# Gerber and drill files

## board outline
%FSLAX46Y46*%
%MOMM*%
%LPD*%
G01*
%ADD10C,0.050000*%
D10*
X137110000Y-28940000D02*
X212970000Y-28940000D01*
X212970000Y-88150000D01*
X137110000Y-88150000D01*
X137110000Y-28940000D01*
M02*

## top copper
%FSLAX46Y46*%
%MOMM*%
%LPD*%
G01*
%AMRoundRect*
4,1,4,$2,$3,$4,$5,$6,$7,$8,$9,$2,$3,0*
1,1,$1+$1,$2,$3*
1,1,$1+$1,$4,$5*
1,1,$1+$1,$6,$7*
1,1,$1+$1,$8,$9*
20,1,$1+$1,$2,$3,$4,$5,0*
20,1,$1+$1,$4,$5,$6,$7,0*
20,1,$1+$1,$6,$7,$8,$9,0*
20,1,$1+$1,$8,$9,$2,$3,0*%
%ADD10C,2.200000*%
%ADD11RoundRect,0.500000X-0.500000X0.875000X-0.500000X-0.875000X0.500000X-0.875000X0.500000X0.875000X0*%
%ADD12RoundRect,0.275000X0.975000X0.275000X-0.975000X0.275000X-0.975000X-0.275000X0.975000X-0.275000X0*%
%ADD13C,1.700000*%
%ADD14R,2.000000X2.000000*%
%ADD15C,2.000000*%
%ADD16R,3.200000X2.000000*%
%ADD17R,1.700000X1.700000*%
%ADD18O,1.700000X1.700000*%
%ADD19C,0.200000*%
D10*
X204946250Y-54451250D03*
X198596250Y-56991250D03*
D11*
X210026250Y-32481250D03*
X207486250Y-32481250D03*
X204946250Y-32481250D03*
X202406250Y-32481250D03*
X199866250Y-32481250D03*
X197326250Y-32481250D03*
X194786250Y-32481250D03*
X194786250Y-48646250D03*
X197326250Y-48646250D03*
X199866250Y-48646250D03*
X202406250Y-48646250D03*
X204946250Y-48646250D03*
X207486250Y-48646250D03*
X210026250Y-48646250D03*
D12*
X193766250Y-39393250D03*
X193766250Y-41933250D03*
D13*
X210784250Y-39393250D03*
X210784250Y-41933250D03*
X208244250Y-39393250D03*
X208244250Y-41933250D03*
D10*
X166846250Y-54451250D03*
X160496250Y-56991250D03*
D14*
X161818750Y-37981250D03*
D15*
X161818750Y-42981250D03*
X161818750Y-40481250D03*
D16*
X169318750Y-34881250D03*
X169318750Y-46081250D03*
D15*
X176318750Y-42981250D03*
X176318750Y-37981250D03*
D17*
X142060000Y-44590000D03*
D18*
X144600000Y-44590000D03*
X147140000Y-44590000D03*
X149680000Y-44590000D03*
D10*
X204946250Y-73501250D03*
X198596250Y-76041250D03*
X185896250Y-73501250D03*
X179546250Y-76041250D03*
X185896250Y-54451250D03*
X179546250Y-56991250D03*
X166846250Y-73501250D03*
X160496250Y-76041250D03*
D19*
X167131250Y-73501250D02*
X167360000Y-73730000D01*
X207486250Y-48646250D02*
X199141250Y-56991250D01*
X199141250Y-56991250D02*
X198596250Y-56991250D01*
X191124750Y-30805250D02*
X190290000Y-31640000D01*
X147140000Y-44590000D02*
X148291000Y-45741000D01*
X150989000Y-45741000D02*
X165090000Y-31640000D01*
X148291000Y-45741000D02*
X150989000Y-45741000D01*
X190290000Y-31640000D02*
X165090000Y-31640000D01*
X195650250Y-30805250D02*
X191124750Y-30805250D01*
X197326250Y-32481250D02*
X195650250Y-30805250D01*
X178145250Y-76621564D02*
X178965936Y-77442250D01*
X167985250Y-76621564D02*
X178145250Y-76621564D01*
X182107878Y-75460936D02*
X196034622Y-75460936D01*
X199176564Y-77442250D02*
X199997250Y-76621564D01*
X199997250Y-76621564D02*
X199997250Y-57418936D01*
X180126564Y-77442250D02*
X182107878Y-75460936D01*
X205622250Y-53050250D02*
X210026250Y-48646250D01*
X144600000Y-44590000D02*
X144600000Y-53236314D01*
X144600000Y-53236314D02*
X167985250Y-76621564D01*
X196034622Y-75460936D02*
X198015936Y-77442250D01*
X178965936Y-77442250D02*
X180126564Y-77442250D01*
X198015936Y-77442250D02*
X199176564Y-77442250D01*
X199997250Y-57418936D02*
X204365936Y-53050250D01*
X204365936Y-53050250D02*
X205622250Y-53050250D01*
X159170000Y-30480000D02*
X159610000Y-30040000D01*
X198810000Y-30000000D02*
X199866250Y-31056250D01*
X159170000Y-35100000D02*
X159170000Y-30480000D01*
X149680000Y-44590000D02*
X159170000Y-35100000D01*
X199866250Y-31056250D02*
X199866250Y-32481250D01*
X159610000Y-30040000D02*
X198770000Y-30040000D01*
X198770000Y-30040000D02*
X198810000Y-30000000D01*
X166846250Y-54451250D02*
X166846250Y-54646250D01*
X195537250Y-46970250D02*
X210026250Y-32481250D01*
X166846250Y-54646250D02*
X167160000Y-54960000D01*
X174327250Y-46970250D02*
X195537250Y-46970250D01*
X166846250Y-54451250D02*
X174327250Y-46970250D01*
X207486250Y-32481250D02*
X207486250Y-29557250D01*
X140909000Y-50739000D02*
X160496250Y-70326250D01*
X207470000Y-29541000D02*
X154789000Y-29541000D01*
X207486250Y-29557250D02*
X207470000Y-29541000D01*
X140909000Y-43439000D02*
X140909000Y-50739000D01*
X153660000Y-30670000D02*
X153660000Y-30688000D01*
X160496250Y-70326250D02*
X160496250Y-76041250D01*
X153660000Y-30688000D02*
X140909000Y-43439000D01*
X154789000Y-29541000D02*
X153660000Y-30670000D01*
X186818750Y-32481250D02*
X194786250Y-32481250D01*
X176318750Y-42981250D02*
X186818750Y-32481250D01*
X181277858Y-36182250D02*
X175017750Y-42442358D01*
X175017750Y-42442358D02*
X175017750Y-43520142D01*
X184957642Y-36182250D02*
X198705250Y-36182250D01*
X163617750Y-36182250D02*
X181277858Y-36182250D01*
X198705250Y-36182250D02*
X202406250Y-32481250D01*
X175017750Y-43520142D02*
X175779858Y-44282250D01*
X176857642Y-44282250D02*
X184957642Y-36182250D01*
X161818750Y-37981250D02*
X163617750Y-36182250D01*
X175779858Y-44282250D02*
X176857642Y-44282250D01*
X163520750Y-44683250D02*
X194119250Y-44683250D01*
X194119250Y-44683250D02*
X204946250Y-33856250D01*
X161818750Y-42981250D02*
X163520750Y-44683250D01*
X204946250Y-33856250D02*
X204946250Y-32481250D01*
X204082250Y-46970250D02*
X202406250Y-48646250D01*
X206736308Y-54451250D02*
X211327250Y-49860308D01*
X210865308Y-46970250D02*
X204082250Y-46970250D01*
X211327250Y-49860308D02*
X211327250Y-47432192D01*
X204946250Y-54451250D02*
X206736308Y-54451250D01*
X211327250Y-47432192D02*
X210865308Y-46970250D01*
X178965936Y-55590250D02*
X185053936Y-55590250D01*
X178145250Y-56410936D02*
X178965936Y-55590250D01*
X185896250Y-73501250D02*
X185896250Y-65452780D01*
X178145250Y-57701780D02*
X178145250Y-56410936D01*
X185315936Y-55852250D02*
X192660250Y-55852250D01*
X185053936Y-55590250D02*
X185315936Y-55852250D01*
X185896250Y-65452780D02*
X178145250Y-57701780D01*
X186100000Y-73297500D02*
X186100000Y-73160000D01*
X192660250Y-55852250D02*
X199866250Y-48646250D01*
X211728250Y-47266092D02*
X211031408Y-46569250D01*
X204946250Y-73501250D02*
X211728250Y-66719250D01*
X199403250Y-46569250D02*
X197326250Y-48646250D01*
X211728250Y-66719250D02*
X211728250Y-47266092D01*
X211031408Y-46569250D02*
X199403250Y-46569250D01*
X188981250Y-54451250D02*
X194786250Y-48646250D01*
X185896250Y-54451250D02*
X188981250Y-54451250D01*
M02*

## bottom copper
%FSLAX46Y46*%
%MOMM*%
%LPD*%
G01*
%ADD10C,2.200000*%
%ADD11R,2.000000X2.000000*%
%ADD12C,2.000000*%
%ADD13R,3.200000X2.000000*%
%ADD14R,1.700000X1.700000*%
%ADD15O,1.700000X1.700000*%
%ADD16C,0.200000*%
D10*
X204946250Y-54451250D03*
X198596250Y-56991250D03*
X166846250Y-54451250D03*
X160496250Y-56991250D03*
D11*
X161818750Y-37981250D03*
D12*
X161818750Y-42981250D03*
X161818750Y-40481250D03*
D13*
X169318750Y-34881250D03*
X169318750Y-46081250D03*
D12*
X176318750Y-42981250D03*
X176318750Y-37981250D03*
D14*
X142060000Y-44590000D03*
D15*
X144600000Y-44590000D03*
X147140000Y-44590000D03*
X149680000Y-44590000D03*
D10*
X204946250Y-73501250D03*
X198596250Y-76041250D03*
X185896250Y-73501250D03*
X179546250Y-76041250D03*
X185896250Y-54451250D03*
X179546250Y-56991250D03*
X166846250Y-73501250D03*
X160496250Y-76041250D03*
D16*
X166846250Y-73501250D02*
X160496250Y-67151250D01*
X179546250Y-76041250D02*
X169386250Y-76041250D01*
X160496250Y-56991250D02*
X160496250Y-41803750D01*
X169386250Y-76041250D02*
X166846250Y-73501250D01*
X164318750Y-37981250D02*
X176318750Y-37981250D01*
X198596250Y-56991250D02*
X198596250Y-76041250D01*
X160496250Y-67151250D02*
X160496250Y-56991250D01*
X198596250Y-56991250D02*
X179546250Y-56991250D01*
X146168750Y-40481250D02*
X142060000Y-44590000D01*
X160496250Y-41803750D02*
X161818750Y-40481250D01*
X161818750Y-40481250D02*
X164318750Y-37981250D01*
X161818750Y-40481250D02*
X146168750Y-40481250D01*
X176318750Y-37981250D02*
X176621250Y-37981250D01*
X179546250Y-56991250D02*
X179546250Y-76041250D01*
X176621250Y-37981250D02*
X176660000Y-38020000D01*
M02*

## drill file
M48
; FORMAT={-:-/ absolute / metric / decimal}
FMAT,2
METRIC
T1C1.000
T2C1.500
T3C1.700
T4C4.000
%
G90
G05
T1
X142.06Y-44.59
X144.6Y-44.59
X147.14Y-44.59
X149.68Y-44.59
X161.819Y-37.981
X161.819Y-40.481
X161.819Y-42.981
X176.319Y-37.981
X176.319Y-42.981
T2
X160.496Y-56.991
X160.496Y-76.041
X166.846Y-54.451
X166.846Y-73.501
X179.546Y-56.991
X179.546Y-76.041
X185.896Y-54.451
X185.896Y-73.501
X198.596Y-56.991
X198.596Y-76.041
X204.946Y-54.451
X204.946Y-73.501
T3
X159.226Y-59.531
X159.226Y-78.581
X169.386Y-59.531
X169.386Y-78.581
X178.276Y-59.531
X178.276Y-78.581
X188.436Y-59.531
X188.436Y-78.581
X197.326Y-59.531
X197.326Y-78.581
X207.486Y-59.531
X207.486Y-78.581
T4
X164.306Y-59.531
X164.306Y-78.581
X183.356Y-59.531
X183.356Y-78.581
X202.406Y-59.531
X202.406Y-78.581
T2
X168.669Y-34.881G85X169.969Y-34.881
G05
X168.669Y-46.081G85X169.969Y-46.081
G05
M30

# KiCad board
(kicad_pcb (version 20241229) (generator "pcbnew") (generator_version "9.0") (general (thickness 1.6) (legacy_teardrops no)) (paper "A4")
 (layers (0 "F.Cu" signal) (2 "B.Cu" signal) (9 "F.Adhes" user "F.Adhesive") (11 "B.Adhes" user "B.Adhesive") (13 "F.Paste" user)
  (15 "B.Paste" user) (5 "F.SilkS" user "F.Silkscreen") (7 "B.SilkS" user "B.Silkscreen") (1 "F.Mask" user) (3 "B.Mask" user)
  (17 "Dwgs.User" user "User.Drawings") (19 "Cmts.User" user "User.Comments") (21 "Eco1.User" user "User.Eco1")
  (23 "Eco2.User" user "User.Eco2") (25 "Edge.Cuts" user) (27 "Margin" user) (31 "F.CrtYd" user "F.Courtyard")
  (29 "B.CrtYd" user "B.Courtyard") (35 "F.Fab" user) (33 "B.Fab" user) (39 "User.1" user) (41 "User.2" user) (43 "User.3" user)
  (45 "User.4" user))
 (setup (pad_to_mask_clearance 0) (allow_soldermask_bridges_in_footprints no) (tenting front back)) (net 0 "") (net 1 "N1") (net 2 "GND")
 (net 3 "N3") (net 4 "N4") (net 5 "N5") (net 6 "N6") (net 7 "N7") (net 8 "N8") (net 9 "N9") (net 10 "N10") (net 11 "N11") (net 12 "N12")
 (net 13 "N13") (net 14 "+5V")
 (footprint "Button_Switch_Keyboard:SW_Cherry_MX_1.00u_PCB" (layer "F.Cu") (at 204.94625 54.45125)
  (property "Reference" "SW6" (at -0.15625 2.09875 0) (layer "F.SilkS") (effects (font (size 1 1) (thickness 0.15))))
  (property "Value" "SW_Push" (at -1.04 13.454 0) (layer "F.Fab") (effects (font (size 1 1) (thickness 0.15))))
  (pad "" np_thru_hole circle (at -7.62 5.08) (size 1.7 1.7) (drill 1.7) (layers "*.Cu" "*.Mask"))
  (pad "" np_thru_hole circle (at -2.54 5.08) (size 4 4) (drill 4) (layers "*.Cu" "*.Mask"))
  (pad "" np_thru_hole circle (at 2.54 5.08) (size 1.7 1.7) (drill 1.7) (layers "*.Cu" "*.Mask"))
  (pad "1" thru_hole circle (at 0 0) (size 2.2 2.2) (drill 1.5) (layers "*.Cu" "*.Mask") (remove_unused_layers no) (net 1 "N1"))
  (pad "2" thru_hole circle (at -6.35 2.54) (size 2.2 2.2) (drill 1.5) (layers "*.Cu" "*.Mask") (remove_unused_layers no) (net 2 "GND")))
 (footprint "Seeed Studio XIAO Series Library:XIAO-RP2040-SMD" (layer "F.Cu") (at 202.40625 40.48125 -90)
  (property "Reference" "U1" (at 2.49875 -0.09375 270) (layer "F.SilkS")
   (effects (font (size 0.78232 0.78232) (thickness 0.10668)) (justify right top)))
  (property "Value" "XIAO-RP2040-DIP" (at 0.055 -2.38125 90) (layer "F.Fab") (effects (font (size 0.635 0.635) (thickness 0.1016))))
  (pad "1" smd roundrect (at -8 -7.62 270) (size 2.75 2) (layers "F.Cu" "F.Mask" "F.Paste") (roundrect_rratio 0.25) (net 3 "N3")
   (solder_mask_margin 0.0508) (thermal_bridge_angle 45))
  (pad "2" smd roundrect (at -8 -5.08 270) (size 2.75 2) (layers "F.Cu" "F.Mask" "F.Paste") (roundrect_rratio 0.25) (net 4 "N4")
   (solder_mask_margin 0.0508) (thermal_bridge_angle 45))
  (pad "3" smd roundrect (at -8 -2.54 270) (size 2.75 2) (layers "F.Cu" "F.Mask" "F.Paste") (roundrect_rratio 0.25) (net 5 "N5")
   (solder_mask_margin 0.0508) (thermal_bridge_angle 45))
  (pad "4" smd roundrect (at -8 0 270) (size 2.75 2) (layers "F.Cu" "F.Mask" "F.Paste") (roundrect_rratio 0.25) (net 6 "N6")
   (solder_mask_margin 0.0508) (thermal_bridge_angle 45))
  (pad "5" smd roundrect (at -8 2.54 270) (size 2.75 2) (layers "F.Cu" "F.Mask" "F.Paste") (roundrect_rratio 0.25) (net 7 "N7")
   (solder_mask_margin 0.0508) (thermal_bridge_angle 45))
  (pad "6" smd roundrect (at -8 5.08 270) (size 2.75 2) (layers "F.Cu" "F.Mask" "F.Paste") (roundrect_rratio 0.25) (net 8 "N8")
   (solder_mask_margin 0.0508) (thermal_bridge_angle 45))
  (pad "7" smd roundrect (at -8 7.62 270) (size 2.75 2) (layers "F.Cu" "F.Mask" "F.Paste") (roundrect_rratio 0.25) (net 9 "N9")
   (solder_mask_margin 0.0508) (thermal_bridge_angle 45))
  (pad "8" smd roundrect (at 8.165 7.62 270) (size 2.75 2) (layers "F.Cu" "F.Mask" "F.Paste") (roundrect_rratio 0.25) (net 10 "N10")
   (solder_mask_margin 0.0508) (thermal_bridge_angle 45))
  (pad "9" smd roundrect (at 8.165 5.08 270) (size 2.75 2) (layers "F.Cu" "F.Mask" "F.Paste") (roundrect_rratio 0.25) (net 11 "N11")
   (solder_mask_margin 0.0508) (thermal_bridge_angle 45))
  (pad "10" smd roundrect (at 8.165 2.54 270) (size 2.75 2) (layers "F.Cu" "F.Mask" "F.Paste") (roundrect_rratio 0.25) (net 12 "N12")
   (solder_mask_margin 0.0508) (thermal_bridge_angle 45))
  (pad "11" smd roundrect (at 8.165 0 270) (size 2.75 2) (layers "F.Cu" "F.Mask" "F.Paste") (roundrect_rratio 0.25) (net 1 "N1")
   (solder_mask_margin 0.0508) (thermal_bridge_angle 45))
  (pad "12" smd roundrect (at 8.165 -2.54 270) (size 2.75 2) (layers "F.Cu" "F.Mask" "F.Paste") (roundrect_rratio 0.25) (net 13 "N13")
   (solder_mask_margin 0.0508) (thermal_bridge_angle 45))
  (pad "13" smd roundrect (at 8.165 -5.08 270) (size 2.75 2) (layers "F.Cu" "F.Mask" "F.Paste") (roundrect_rratio 0.25) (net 2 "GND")
   (solder_mask_margin 0.0508) (thermal_bridge_angle 45))
  (pad "14" smd roundrect (at 8.165 -7.62 270) (size 2.75 2) (layers "F.Cu" "F.Mask" "F.Paste") (roundrect_rratio 0.25) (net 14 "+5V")
   (solder_mask_margin 0.0508) (thermal_bridge_angle 45))
  (pad "15" smd roundrect (at -1.088 8.64 180) (size 2.5 1.1) (layers "F.Cu" "F.Mask" "F.Paste") (roundrect_rratio 0.25)
   (thermal_bridge_angle 45))
  (pad "16" smd roundrect (at 1.452 8.64 180) (size 2.5 1.1) (layers "F.Cu" "F.Mask" "F.Paste") (roundrect_rratio 0.25)
   (thermal_bridge_angle 45))
  (pad "17" smd circle (at -1.088 -8.378 270) (size 1.7 1.7) (layers "F.Cu" "F.Mask" "F.Paste"))
  (pad "18" smd circle (at 1.452 -8.378 270) (size 1.7 1.7) (layers "F.Cu" "F.Mask" "F.Paste"))
  (pad "19" smd circle (at -1.088 -5.838 270) (size 1.7 1.7) (layers "F.Cu" "F.Mask" "F.Paste"))
  (pad "20" smd circle (at 1.452 -5.838 270) (size 1.7 1.7) (layers "F.Cu" "F.Mask" "F.Paste")))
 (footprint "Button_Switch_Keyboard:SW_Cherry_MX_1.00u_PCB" (layer "F.Cu") (at 166.84625 54.45125)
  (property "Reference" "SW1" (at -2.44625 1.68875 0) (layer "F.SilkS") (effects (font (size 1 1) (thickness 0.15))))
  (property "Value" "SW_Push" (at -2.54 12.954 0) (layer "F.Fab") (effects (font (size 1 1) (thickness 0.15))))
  (pad "" np_thru_hole circle (at -7.62 5.08) (size 1.7 1.7) (drill 1.7) (layers "*.Cu" "*.Mask"))
  (pad "" np_thru_hole circle (at -2.54 5.08) (size 4 4) (drill 4) (layers "*.Cu" "*.Mask"))
  (pad "" np_thru_hole circle (at 2.54 5.08) (size 1.7 1.7) (drill 1.7) (layers "*.Cu" "*.Mask"))
  (pad "1" thru_hole circle (at 0 0) (size 2.2 2.2) (drill 1.5) (layers "*.Cu" "*.Mask") (remove_unused_layers no) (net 3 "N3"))
  (pad "2" thru_hole circle (at -6.35 2.54) (size 2.2 2.2) (drill 1.5) (layers "*.Cu" "*.Mask") (remove_unused_layers no) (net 2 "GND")))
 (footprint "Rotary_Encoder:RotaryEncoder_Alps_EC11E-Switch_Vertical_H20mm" (layer "F.Cu") (at 161.81875 37.98125)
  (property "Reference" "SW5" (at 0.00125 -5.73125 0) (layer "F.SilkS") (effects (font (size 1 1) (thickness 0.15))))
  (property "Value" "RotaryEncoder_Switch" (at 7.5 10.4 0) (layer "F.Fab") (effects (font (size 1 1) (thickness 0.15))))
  (pad "A" thru_hole rect (at 0 0) (size 2 2) (drill 1) (layers "*.Cu" "*.Mask") (remove_unused_layers no) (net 6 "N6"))
  (pad "B" thru_hole circle (at 0 5) (size 2 2) (drill 1) (layers "*.Cu" "*.Mask") (remove_unused_layers no) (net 5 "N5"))
  (pad "C" thru_hole circle (at 0 2.5) (size 2 2) (drill 1) (layers "*.Cu" "*.Mask") (remove_unused_layers no) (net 2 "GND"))
  (pad "MP" thru_hole rect (at 7.5 -3.1) (size 3.2 2) (drill oval 2.8 1.5) (layers "*.Cu" "*.Mask") (remove_unused_layers no))
  (pad "MP" thru_hole rect (at 7.5 8.1) (size 3.2 2) (drill oval 2.8 1.5) (layers "*.Cu" "*.Mask") (remove_unused_layers no))
  (pad "S1" thru_hole circle (at 14.5 5) (size 2 2) (drill 1) (layers "*.Cu" "*.Mask") (remove_unused_layers no) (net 9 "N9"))
  (pad "S2" thru_hole circle (at 14.5 0) (size 2 2) (drill 1) (layers "*.Cu" "*.Mask") (remove_unused_layers no) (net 2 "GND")))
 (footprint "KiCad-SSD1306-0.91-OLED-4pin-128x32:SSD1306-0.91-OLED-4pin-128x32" (layer "F.Cu") (at 139.87 81.09 90)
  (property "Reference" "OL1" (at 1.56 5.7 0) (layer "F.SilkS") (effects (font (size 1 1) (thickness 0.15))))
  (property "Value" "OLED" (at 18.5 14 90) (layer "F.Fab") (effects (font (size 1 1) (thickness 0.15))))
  (pad "1" thru_hole rect (at 36.5 2.19 90) (size 1.7 1.7) (drill 1) (layers "*.Cu" "*.Mask") (remove_unused_layers no) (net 2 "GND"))
  (pad "2" thru_hole oval (at 36.5 4.73 90) (size 1.7 1.7) (drill 1) (layers "*.Cu" "*.Mask") (remove_unused_layers no) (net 14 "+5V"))
  (pad "3" thru_hole oval (at 36.5 7.27 90) (size 1.7 1.7) (drill 1) (layers "*.Cu" "*.Mask") (remove_unused_layers no) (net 8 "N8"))
  (pad "4" thru_hole oval (at 36.5 9.81 90) (size 1.7 1.7) (drill 1) (layers "*.Cu" "*.Mask") (remove_unused_layers no) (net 7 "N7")))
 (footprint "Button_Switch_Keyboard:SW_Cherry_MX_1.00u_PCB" (layer "F.Cu") (at 204.94625 73.50125)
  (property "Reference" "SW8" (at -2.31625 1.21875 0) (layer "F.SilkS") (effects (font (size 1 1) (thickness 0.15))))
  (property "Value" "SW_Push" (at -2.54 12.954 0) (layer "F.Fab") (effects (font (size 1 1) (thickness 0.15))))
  (pad "" np_thru_hole circle (at -7.62 5.08) (size 1.7 1.7) (drill 1.7) (layers "*.Cu" "*.Mask"))
  (pad "" np_thru_hole circle (at -2.54 5.08) (size 4 4) (drill 4) (layers "*.Cu" "*.Mask"))
  (pad "" np_thru_hole circle (at 2.54 5.08) (size 1.7 1.7) (drill 1.7) (layers "*.Cu" "*.Mask"))
  (pad "1" thru_hole circle (at 0 0) (size 2.2 2.2) (drill 1.5) (layers "*.Cu" "*.Mask") (remove_unused_layers no) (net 11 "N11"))
  (pad "2" thru_hole circle (at -6.35 2.54) (size 2.2 2.2) (drill 1.5) (layers "*.Cu" "*.Mask") (remove_unused_layers no) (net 2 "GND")))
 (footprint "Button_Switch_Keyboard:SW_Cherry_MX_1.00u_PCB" (layer "F.Cu") (at 185.89625 73.50125)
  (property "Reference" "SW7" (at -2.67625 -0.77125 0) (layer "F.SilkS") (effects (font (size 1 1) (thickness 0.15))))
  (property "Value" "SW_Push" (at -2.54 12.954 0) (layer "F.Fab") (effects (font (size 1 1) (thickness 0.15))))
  (pad "" np_thru_hole circle (at -7.62 5.08) (size 1.7 1.7) (drill 1.7) (layers "*.Cu" "*.Mask"))
  (pad "" np_thru_hole circle (at -2.54 5.08) (size 4 4) (drill 4) (layers "*.Cu" "*.Mask"))
  (pad "" np_thru_hole circle (at 2.54 5.08) (size 1.7 1.7) (drill 1.7) (layers "*.Cu" "*.Mask"))
  (pad "1" thru_hole circle (at 0 0) (size 2.2 2.2) (drill 1.5) (layers "*.Cu" "*.Mask") (remove_unused_layers no) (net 12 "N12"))
  (pad "2" thru_hole circle (at -6.35 2.54) (size 2.2 2.2) (drill 1.5) (layers "*.Cu" "*.Mask") (remove_unused_layers no) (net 2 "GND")))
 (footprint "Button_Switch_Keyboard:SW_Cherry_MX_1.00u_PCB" (layer "F.Cu") (at 185.89625 54.45125)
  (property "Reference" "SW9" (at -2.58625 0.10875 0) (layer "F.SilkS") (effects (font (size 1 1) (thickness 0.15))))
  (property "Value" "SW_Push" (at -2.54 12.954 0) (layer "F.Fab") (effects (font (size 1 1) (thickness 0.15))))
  (pad "" np_thru_hole circle (at -7.62 5.08) (size 1.7 1.7) (drill 1.7) (layers "*.Cu" "*.Mask"))
  (pad "" np_thru_hole circle (at -2.54 5.08) (size 4 4) (drill 4) (layers "*.Cu" "*.Mask"))
  (pad "" np_thru_hole circle (at 2.54 5.08) (size 1.7 1.7) (drill 1.7) (layers "*.Cu" "*.Mask"))
  (pad "1" thru_hole circle (at 0 0) (size 2.2 2.2) (drill 1.5) (layers "*.Cu" "*.Mask") (remove_unused_layers no) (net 10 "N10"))
  (pad "2" thru_hole circle (at -6.35 2.54) (size 2.2 2.2) (drill 1.5) (layers "*.Cu" "*.Mask") (remove_unused_layers no) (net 2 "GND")))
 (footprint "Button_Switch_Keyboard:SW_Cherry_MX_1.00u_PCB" (layer "F.Cu") (at 166.84625 73.50125)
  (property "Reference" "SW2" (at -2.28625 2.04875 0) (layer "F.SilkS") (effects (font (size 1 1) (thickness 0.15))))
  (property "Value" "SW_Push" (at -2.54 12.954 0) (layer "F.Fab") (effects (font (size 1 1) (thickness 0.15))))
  (pad "" np_thru_hole circle (at -7.62 5.08) (size 1.7 1.7) (drill 1.7) (layers "*.Cu" "*.Mask"))
  (pad "" np_thru_hole circle (at -2.54 5.08) (size 4 4) (drill 4) (layers "*.Cu" "*.Mask"))
  (pad "" np_thru_hole circle (at 2.54 5.08) (size 1.7 1.7) (drill 1.7) (layers "*.Cu" "*.Mask"))
  (pad "1" thru_hole circle (at 0 0) (size 2.2 2.2) (drill 1.5) (layers "*.Cu" "*.Mask") (remove_unused_layers no) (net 2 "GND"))
  (pad "2" thru_hole circle (at -6.35 2.54) (size 2.2 2.2) (drill 1.5) (layers "*.Cu" "*.Mask") (remove_unused_layers no) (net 4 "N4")))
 (gr_rect (start 137.11 28.94) (end 212.97 88.15) (stroke (width 0.05) (type default)) (fill no) (layer "Edge.Cuts"))
 (segment (start 167.13125 73.50125) (end 167.36 73.73) (width 0.2) (layer "F.Cu") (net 2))
 (segment (start 207.48625 48.64625) (end 199.14125 56.99125) (width 0.2) (layer "F.Cu") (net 2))
 (segment (start 199.14125 56.99125) (end 198.59625 56.99125) (width 0.2) (layer "F.Cu") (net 2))
 (segment (start 166.84625 73.50125) (end 160.49625 67.15125) (width 0.2) (layer "B.Cu") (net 2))
 (segment (start 179.54625 76.04125) (end 169.38625 76.04125) (width 0.2) (layer "B.Cu") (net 2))
 (segment (start 160.49625 56.99125) (end 160.49625 41.80375) (width 0.2) (layer "B.Cu") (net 2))
 (segment (start 169.38625 76.04125) (end 166.84625 73.50125) (width 0.2) (layer "B.Cu") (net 2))
 (segment (start 164.31875 37.98125) (end 176.31875 37.98125) (width 0.2) (layer "B.Cu") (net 2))
 (segment (start 198.59625 56.99125) (end 198.59625 76.04125) (width 0.2) (layer "B.Cu") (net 2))
 (segment (start 160.49625 67.15125) (end 160.49625 56.99125) (width 0.2) (layer "B.Cu") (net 2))
 (segment (start 198.59625 56.99125) (end 179.54625 56.99125) (width 0.2) (layer "B.Cu") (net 2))
 (segment (start 146.16875 40.48125) (end 142.06 44.59) (width 0.2) (layer "B.Cu") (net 2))
 (segment (start 160.49625 41.80375) (end 161.81875 40.48125) (width 0.2) (layer "B.Cu") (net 2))
 (segment (start 161.81875 40.48125) (end 164.31875 37.98125) (width 0.2) (layer "B.Cu") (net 2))
 (segment (start 161.81875 40.48125) (end 146.16875 40.48125) (width 0.2) (layer "B.Cu") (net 2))
 (segment (start 176.31875 37.98125) (end 176.62125 37.98125) (width 0.2) (layer "B.Cu") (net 2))
 (segment (start 179.54625 56.99125) (end 179.54625 76.04125) (width 0.2) (layer "B.Cu") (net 2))
 (segment (start 176.62125 37.98125) (end 176.66 38.02) (width 0.2) (layer "B.Cu") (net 2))
 (segment (start 191.12475 30.80525) (end 190.29 31.64) (width 0.2) (layer "F.Cu") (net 8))
 (segment (start 147.14 44.59) (end 148.291 45.741) (width 0.2) (layer "F.Cu") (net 8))
 (segment (start 150.989 45.741) (end 165.09 31.64) (width 0.2) (layer "F.Cu") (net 8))
 (segment (start 148.291 45.741) (end 150.989 45.741) (width 0.2) (layer "F.Cu") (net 8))
 (segment (start 190.29 31.64) (end 165.09 31.64) (width 0.2) (layer "F.Cu") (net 8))
 (segment (start 195.65025 30.80525) (end 191.12475 30.80525) (width 0.2) (layer "F.Cu") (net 8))
 (segment (start 197.32625 32.48125) (end 195.65025 30.80525) (width 0.2) (layer "F.Cu") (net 8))
 (segment (start 178.14525 76.621564) (end 178.965936 77.44225) (width 0.2) (layer "F.Cu") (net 14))
 (segment (start 167.98525 76.621564) (end 178.14525 76.621564) (width 0.2) (layer "F.Cu") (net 14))
 (segment (start 182.107878 75.460936) (end 196.034622 75.460936) (width 0.2) (layer "F.Cu") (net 14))
 (segment (start 199.176564 77.44225) (end 199.99725 76.621564) (width 0.2) (layer "F.Cu") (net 14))
 (segment (start 199.99725 76.621564) (end 199.99725 57.418936) (width 0.2) (layer "F.Cu") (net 14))
 (segment (start 180.126564 77.44225) (end 182.107878 75.460936) (width 0.2) (layer "F.Cu") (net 14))
 (segment (start 205.62225 53.05025) (end 210.02625 48.64625) (width 0.2) (layer "F.Cu") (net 14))
 (segment (start 144.6 44.59) (end 144.6 53.236314) (width 0.2) (layer "F.Cu") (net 14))
 (segment (start 144.6 53.236314) (end 167.98525 76.621564) (width 0.2) (layer "F.Cu") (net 14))
 (segment (start 196.034622 75.460936) (end 198.015936 77.44225) (width 0.2) (layer "F.Cu") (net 14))
 (segment (start 178.965936 77.44225) (end 180.126564 77.44225) (width 0.2) (layer "F.Cu") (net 14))
 (segment (start 198.015936 77.44225) (end 199.176564 77.44225) (width 0.2) (layer "F.Cu") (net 14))
 (segment (start 199.99725 57.418936) (end 204.365936 53.05025) (width 0.2) (layer "F.Cu") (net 14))
 (segment (start 204.365936 53.05025) (end 205.62225 53.05025) (width 0.2) (layer "F.Cu") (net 14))
 (segment (start 159.17 30.48) (end 159.61 30.04) (width 0.2) (layer "F.Cu") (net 7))
 (segment (start 198.81 30) (end 199.86625 31.05625) (width 0.2) (layer "F.Cu") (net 7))
 (segment (start 159.17 35.1) (end 159.17 30.48) (width 0.2) (layer "F.Cu") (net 7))
 (segment (start 149.68 44.59) (end 159.17 35.1) (width 0.2) (layer "F.Cu") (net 7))
 (segment (start 199.86625 31.05625) (end 199.86625 32.48125) (width 0.2) (layer "F.Cu") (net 7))
 (segment (start 159.61 30.04) (end 198.77 30.04) (width 0.2) (layer "F.Cu") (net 7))
 (segment (start 198.77 30.04) (end 198.81 30) (width 0.2) (layer "F.Cu") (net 7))
 (segment (start 166.84625 54.45125) (end 166.84625 54.64625) (width 0.2) (layer "F.Cu") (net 3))
 (segment (start 195.53725 46.97025) (end 210.02625 32.48125) (width 0.2) (layer "F.Cu") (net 3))
 (segment (start 166.84625 54.64625) (end 167.16 54.96) (width 0.2) (layer "F.Cu") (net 3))
 (segment (start 174.32725 46.97025) (end 195.53725 46.97025) (width 0.2) (layer "F.Cu") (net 3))
 (segment (start 166.84625 54.45125) (end 174.32725 46.97025) (width 0.2) (layer "F.Cu") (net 3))
 (segment (start 207.48625 32.48125) (end 207.48625 29.55725) (width 0.2) (layer "F.Cu") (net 4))
 (segment (start 140.909 50.739) (end 160.49625 70.32625) (width 0.2) (layer "F.Cu") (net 4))
 (segment (start 207.47 29.541) (end 154.789 29.541) (width 0.2) (layer "F.Cu") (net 4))
 (segment (start 207.48625 29.55725) (end 207.47 29.541) (width 0.2) (layer "F.Cu") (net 4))
 (segment (start 140.909 43.439) (end 140.909 50.739) (width 0.2) (layer "F.Cu") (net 4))
 (segment (start 153.66 30.67) (end 153.66 30.688) (width 0.2) (layer "F.Cu") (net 4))
 (segment (start 160.49625 70.32625) (end 160.49625 76.04125) (width 0.2) (layer "F.Cu") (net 4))
 (segment (start 153.66 30.688) (end 140.909 43.439) (width 0.2) (layer "F.Cu") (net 4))
 (segment (start 154.789 29.541) (end 153.66 30.67) (width 0.2) (layer "F.Cu") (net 4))
 (segment (start 186.81875 32.48125) (end 194.78625 32.48125) (width 0.2) (layer "F.Cu") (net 9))
 (segment (start 176.31875 42.98125) (end 186.81875 32.48125) (width 0.2) (layer "F.Cu") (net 9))
 (segment (start 181.277858 36.18225) (end 175.01775 42.442358) (width 0.2) (layer "F.Cu") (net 6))
 (segment (start 175.01775 42.442358) (end 175.01775 43.520142) (width 0.2) (layer "F.Cu") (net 6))
 (segment (start 184.957642 36.18225) (end 198.70525 36.18225) (width 0.2) (layer "F.Cu") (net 6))
 (segment (start 163.61775 36.18225) (end 181.277858 36.18225) (width 0.2) (layer "F.Cu") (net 6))
 (segment (start 198.70525 36.18225) (end 202.40625 32.48125) (width 0.2) (layer "F.Cu") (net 6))
 (segment (start 175.01775 43.520142) (end 175.779858 44.28225) (width 0.2) (layer "F.Cu") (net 6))
 (segment (start 176.857642 44.28225) (end 184.957642 36.18225) (width 0.2) (layer "F.Cu") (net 6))
 (segment (start 161.81875 37.98125) (end 163.61775 36.18225) (width 0.2) (layer "F.Cu") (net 6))
 (segment (start 175.779858 44.28225) (end 176.857642 44.28225) (width 0.2) (layer "F.Cu") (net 6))
 (segment (start 163.52075 44.68325) (end 194.11925 44.68325) (width 0.2) (layer "F.Cu") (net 5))
 (segment (start 194.11925 44.68325) (end 204.94625 33.85625) (width 0.2) (layer "F.Cu") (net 5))
 (segment (start 161.81875 42.98125) (end 163.52075 44.68325) (width 0.2) (layer "F.Cu") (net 5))
 (segment (start 204.94625 33.85625) (end 204.94625 32.48125) (width 0.2) (layer "F.Cu") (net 5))
 (segment (start 204.08225 46.97025) (end 202.40625 48.64625) (width 0.2) (layer "F.Cu") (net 1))
 (segment (start 206.736308 54.45125) (end 211.32725 49.860308) (width 0.2) (layer "F.Cu") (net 1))
 (segment (start 210.865308 46.97025) (end 204.08225 46.97025) (width 0.2) (layer "F.Cu") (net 1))
 (segment (start 211.32725 49.860308) (end 211.32725 47.432192) (width 0.2) (layer "F.Cu") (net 1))
 (segment (start 204.94625 54.45125) (end 206.736308 54.45125) (width 0.2) (layer "F.Cu") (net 1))
 (segment (start 211.32725 47.432192) (end 210.865308 46.97025) (width 0.2) (layer "F.Cu") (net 1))
 (segment (start 178.965936 55.59025) (end 185.053936 55.59025) (width 0.2) (layer "F.Cu") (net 12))
 (segment (start 178.14525 56.410936) (end 178.965936 55.59025) (width 0.2) (layer "F.Cu") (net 12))
 (segment (start 185.89625 73.50125) (end 185.89625 65.45278) (width 0.2) (layer "F.Cu") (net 12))
 (segment (start 178.14525 57.70178) (end 178.14525 56.410936) (width 0.2) (layer "F.Cu") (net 12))
 (segment (start 185.315936 55.85225) (end 192.66025 55.85225) (width 0.2) (layer "F.Cu") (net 12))
 (segment (start 185.053936 55.59025) (end 185.315936 55.85225) (width 0.2) (layer "F.Cu") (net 12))
 (segment (start 185.89625 65.45278) (end 178.14525 57.70178) (width 0.2) (layer "F.Cu") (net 12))
 (segment (start 186.1 73.2975) (end 186.1 73.16) (width 0.2) (layer "F.Cu") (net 12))
 (segment (start 192.66025 55.85225) (end 199.86625 48.64625) (width 0.2) (layer "F.Cu") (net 12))
 (segment (start 211.72825 47.266092) (end 211.031408 46.56925) (width 0.2) (layer "F.Cu") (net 11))
 (segment (start 204.94625 73.50125) (end 211.72825 66.71925) (width 0.2) (layer "F.Cu") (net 11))
 (segment (start 199.40325 46.56925) (end 197.32625 48.64625) (width 0.2) (layer "F.Cu") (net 11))
 (segment (start 211.72825 66.71925) (end 211.72825 47.266092) (width 0.2) (layer "F.Cu") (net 11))
 (segment (start 211.031408 46.56925) (end 199.40325 46.56925) (width 0.2) (layer "F.Cu") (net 11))
 (segment (start 188.98125 54.45125) (end 194.78625 48.64625) (width 0.2) (layer "F.Cu") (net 10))
 (segment (start 185.89625 54.45125) (end 188.98125 54.45125) (width 0.2) (layer "F.Cu") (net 10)))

